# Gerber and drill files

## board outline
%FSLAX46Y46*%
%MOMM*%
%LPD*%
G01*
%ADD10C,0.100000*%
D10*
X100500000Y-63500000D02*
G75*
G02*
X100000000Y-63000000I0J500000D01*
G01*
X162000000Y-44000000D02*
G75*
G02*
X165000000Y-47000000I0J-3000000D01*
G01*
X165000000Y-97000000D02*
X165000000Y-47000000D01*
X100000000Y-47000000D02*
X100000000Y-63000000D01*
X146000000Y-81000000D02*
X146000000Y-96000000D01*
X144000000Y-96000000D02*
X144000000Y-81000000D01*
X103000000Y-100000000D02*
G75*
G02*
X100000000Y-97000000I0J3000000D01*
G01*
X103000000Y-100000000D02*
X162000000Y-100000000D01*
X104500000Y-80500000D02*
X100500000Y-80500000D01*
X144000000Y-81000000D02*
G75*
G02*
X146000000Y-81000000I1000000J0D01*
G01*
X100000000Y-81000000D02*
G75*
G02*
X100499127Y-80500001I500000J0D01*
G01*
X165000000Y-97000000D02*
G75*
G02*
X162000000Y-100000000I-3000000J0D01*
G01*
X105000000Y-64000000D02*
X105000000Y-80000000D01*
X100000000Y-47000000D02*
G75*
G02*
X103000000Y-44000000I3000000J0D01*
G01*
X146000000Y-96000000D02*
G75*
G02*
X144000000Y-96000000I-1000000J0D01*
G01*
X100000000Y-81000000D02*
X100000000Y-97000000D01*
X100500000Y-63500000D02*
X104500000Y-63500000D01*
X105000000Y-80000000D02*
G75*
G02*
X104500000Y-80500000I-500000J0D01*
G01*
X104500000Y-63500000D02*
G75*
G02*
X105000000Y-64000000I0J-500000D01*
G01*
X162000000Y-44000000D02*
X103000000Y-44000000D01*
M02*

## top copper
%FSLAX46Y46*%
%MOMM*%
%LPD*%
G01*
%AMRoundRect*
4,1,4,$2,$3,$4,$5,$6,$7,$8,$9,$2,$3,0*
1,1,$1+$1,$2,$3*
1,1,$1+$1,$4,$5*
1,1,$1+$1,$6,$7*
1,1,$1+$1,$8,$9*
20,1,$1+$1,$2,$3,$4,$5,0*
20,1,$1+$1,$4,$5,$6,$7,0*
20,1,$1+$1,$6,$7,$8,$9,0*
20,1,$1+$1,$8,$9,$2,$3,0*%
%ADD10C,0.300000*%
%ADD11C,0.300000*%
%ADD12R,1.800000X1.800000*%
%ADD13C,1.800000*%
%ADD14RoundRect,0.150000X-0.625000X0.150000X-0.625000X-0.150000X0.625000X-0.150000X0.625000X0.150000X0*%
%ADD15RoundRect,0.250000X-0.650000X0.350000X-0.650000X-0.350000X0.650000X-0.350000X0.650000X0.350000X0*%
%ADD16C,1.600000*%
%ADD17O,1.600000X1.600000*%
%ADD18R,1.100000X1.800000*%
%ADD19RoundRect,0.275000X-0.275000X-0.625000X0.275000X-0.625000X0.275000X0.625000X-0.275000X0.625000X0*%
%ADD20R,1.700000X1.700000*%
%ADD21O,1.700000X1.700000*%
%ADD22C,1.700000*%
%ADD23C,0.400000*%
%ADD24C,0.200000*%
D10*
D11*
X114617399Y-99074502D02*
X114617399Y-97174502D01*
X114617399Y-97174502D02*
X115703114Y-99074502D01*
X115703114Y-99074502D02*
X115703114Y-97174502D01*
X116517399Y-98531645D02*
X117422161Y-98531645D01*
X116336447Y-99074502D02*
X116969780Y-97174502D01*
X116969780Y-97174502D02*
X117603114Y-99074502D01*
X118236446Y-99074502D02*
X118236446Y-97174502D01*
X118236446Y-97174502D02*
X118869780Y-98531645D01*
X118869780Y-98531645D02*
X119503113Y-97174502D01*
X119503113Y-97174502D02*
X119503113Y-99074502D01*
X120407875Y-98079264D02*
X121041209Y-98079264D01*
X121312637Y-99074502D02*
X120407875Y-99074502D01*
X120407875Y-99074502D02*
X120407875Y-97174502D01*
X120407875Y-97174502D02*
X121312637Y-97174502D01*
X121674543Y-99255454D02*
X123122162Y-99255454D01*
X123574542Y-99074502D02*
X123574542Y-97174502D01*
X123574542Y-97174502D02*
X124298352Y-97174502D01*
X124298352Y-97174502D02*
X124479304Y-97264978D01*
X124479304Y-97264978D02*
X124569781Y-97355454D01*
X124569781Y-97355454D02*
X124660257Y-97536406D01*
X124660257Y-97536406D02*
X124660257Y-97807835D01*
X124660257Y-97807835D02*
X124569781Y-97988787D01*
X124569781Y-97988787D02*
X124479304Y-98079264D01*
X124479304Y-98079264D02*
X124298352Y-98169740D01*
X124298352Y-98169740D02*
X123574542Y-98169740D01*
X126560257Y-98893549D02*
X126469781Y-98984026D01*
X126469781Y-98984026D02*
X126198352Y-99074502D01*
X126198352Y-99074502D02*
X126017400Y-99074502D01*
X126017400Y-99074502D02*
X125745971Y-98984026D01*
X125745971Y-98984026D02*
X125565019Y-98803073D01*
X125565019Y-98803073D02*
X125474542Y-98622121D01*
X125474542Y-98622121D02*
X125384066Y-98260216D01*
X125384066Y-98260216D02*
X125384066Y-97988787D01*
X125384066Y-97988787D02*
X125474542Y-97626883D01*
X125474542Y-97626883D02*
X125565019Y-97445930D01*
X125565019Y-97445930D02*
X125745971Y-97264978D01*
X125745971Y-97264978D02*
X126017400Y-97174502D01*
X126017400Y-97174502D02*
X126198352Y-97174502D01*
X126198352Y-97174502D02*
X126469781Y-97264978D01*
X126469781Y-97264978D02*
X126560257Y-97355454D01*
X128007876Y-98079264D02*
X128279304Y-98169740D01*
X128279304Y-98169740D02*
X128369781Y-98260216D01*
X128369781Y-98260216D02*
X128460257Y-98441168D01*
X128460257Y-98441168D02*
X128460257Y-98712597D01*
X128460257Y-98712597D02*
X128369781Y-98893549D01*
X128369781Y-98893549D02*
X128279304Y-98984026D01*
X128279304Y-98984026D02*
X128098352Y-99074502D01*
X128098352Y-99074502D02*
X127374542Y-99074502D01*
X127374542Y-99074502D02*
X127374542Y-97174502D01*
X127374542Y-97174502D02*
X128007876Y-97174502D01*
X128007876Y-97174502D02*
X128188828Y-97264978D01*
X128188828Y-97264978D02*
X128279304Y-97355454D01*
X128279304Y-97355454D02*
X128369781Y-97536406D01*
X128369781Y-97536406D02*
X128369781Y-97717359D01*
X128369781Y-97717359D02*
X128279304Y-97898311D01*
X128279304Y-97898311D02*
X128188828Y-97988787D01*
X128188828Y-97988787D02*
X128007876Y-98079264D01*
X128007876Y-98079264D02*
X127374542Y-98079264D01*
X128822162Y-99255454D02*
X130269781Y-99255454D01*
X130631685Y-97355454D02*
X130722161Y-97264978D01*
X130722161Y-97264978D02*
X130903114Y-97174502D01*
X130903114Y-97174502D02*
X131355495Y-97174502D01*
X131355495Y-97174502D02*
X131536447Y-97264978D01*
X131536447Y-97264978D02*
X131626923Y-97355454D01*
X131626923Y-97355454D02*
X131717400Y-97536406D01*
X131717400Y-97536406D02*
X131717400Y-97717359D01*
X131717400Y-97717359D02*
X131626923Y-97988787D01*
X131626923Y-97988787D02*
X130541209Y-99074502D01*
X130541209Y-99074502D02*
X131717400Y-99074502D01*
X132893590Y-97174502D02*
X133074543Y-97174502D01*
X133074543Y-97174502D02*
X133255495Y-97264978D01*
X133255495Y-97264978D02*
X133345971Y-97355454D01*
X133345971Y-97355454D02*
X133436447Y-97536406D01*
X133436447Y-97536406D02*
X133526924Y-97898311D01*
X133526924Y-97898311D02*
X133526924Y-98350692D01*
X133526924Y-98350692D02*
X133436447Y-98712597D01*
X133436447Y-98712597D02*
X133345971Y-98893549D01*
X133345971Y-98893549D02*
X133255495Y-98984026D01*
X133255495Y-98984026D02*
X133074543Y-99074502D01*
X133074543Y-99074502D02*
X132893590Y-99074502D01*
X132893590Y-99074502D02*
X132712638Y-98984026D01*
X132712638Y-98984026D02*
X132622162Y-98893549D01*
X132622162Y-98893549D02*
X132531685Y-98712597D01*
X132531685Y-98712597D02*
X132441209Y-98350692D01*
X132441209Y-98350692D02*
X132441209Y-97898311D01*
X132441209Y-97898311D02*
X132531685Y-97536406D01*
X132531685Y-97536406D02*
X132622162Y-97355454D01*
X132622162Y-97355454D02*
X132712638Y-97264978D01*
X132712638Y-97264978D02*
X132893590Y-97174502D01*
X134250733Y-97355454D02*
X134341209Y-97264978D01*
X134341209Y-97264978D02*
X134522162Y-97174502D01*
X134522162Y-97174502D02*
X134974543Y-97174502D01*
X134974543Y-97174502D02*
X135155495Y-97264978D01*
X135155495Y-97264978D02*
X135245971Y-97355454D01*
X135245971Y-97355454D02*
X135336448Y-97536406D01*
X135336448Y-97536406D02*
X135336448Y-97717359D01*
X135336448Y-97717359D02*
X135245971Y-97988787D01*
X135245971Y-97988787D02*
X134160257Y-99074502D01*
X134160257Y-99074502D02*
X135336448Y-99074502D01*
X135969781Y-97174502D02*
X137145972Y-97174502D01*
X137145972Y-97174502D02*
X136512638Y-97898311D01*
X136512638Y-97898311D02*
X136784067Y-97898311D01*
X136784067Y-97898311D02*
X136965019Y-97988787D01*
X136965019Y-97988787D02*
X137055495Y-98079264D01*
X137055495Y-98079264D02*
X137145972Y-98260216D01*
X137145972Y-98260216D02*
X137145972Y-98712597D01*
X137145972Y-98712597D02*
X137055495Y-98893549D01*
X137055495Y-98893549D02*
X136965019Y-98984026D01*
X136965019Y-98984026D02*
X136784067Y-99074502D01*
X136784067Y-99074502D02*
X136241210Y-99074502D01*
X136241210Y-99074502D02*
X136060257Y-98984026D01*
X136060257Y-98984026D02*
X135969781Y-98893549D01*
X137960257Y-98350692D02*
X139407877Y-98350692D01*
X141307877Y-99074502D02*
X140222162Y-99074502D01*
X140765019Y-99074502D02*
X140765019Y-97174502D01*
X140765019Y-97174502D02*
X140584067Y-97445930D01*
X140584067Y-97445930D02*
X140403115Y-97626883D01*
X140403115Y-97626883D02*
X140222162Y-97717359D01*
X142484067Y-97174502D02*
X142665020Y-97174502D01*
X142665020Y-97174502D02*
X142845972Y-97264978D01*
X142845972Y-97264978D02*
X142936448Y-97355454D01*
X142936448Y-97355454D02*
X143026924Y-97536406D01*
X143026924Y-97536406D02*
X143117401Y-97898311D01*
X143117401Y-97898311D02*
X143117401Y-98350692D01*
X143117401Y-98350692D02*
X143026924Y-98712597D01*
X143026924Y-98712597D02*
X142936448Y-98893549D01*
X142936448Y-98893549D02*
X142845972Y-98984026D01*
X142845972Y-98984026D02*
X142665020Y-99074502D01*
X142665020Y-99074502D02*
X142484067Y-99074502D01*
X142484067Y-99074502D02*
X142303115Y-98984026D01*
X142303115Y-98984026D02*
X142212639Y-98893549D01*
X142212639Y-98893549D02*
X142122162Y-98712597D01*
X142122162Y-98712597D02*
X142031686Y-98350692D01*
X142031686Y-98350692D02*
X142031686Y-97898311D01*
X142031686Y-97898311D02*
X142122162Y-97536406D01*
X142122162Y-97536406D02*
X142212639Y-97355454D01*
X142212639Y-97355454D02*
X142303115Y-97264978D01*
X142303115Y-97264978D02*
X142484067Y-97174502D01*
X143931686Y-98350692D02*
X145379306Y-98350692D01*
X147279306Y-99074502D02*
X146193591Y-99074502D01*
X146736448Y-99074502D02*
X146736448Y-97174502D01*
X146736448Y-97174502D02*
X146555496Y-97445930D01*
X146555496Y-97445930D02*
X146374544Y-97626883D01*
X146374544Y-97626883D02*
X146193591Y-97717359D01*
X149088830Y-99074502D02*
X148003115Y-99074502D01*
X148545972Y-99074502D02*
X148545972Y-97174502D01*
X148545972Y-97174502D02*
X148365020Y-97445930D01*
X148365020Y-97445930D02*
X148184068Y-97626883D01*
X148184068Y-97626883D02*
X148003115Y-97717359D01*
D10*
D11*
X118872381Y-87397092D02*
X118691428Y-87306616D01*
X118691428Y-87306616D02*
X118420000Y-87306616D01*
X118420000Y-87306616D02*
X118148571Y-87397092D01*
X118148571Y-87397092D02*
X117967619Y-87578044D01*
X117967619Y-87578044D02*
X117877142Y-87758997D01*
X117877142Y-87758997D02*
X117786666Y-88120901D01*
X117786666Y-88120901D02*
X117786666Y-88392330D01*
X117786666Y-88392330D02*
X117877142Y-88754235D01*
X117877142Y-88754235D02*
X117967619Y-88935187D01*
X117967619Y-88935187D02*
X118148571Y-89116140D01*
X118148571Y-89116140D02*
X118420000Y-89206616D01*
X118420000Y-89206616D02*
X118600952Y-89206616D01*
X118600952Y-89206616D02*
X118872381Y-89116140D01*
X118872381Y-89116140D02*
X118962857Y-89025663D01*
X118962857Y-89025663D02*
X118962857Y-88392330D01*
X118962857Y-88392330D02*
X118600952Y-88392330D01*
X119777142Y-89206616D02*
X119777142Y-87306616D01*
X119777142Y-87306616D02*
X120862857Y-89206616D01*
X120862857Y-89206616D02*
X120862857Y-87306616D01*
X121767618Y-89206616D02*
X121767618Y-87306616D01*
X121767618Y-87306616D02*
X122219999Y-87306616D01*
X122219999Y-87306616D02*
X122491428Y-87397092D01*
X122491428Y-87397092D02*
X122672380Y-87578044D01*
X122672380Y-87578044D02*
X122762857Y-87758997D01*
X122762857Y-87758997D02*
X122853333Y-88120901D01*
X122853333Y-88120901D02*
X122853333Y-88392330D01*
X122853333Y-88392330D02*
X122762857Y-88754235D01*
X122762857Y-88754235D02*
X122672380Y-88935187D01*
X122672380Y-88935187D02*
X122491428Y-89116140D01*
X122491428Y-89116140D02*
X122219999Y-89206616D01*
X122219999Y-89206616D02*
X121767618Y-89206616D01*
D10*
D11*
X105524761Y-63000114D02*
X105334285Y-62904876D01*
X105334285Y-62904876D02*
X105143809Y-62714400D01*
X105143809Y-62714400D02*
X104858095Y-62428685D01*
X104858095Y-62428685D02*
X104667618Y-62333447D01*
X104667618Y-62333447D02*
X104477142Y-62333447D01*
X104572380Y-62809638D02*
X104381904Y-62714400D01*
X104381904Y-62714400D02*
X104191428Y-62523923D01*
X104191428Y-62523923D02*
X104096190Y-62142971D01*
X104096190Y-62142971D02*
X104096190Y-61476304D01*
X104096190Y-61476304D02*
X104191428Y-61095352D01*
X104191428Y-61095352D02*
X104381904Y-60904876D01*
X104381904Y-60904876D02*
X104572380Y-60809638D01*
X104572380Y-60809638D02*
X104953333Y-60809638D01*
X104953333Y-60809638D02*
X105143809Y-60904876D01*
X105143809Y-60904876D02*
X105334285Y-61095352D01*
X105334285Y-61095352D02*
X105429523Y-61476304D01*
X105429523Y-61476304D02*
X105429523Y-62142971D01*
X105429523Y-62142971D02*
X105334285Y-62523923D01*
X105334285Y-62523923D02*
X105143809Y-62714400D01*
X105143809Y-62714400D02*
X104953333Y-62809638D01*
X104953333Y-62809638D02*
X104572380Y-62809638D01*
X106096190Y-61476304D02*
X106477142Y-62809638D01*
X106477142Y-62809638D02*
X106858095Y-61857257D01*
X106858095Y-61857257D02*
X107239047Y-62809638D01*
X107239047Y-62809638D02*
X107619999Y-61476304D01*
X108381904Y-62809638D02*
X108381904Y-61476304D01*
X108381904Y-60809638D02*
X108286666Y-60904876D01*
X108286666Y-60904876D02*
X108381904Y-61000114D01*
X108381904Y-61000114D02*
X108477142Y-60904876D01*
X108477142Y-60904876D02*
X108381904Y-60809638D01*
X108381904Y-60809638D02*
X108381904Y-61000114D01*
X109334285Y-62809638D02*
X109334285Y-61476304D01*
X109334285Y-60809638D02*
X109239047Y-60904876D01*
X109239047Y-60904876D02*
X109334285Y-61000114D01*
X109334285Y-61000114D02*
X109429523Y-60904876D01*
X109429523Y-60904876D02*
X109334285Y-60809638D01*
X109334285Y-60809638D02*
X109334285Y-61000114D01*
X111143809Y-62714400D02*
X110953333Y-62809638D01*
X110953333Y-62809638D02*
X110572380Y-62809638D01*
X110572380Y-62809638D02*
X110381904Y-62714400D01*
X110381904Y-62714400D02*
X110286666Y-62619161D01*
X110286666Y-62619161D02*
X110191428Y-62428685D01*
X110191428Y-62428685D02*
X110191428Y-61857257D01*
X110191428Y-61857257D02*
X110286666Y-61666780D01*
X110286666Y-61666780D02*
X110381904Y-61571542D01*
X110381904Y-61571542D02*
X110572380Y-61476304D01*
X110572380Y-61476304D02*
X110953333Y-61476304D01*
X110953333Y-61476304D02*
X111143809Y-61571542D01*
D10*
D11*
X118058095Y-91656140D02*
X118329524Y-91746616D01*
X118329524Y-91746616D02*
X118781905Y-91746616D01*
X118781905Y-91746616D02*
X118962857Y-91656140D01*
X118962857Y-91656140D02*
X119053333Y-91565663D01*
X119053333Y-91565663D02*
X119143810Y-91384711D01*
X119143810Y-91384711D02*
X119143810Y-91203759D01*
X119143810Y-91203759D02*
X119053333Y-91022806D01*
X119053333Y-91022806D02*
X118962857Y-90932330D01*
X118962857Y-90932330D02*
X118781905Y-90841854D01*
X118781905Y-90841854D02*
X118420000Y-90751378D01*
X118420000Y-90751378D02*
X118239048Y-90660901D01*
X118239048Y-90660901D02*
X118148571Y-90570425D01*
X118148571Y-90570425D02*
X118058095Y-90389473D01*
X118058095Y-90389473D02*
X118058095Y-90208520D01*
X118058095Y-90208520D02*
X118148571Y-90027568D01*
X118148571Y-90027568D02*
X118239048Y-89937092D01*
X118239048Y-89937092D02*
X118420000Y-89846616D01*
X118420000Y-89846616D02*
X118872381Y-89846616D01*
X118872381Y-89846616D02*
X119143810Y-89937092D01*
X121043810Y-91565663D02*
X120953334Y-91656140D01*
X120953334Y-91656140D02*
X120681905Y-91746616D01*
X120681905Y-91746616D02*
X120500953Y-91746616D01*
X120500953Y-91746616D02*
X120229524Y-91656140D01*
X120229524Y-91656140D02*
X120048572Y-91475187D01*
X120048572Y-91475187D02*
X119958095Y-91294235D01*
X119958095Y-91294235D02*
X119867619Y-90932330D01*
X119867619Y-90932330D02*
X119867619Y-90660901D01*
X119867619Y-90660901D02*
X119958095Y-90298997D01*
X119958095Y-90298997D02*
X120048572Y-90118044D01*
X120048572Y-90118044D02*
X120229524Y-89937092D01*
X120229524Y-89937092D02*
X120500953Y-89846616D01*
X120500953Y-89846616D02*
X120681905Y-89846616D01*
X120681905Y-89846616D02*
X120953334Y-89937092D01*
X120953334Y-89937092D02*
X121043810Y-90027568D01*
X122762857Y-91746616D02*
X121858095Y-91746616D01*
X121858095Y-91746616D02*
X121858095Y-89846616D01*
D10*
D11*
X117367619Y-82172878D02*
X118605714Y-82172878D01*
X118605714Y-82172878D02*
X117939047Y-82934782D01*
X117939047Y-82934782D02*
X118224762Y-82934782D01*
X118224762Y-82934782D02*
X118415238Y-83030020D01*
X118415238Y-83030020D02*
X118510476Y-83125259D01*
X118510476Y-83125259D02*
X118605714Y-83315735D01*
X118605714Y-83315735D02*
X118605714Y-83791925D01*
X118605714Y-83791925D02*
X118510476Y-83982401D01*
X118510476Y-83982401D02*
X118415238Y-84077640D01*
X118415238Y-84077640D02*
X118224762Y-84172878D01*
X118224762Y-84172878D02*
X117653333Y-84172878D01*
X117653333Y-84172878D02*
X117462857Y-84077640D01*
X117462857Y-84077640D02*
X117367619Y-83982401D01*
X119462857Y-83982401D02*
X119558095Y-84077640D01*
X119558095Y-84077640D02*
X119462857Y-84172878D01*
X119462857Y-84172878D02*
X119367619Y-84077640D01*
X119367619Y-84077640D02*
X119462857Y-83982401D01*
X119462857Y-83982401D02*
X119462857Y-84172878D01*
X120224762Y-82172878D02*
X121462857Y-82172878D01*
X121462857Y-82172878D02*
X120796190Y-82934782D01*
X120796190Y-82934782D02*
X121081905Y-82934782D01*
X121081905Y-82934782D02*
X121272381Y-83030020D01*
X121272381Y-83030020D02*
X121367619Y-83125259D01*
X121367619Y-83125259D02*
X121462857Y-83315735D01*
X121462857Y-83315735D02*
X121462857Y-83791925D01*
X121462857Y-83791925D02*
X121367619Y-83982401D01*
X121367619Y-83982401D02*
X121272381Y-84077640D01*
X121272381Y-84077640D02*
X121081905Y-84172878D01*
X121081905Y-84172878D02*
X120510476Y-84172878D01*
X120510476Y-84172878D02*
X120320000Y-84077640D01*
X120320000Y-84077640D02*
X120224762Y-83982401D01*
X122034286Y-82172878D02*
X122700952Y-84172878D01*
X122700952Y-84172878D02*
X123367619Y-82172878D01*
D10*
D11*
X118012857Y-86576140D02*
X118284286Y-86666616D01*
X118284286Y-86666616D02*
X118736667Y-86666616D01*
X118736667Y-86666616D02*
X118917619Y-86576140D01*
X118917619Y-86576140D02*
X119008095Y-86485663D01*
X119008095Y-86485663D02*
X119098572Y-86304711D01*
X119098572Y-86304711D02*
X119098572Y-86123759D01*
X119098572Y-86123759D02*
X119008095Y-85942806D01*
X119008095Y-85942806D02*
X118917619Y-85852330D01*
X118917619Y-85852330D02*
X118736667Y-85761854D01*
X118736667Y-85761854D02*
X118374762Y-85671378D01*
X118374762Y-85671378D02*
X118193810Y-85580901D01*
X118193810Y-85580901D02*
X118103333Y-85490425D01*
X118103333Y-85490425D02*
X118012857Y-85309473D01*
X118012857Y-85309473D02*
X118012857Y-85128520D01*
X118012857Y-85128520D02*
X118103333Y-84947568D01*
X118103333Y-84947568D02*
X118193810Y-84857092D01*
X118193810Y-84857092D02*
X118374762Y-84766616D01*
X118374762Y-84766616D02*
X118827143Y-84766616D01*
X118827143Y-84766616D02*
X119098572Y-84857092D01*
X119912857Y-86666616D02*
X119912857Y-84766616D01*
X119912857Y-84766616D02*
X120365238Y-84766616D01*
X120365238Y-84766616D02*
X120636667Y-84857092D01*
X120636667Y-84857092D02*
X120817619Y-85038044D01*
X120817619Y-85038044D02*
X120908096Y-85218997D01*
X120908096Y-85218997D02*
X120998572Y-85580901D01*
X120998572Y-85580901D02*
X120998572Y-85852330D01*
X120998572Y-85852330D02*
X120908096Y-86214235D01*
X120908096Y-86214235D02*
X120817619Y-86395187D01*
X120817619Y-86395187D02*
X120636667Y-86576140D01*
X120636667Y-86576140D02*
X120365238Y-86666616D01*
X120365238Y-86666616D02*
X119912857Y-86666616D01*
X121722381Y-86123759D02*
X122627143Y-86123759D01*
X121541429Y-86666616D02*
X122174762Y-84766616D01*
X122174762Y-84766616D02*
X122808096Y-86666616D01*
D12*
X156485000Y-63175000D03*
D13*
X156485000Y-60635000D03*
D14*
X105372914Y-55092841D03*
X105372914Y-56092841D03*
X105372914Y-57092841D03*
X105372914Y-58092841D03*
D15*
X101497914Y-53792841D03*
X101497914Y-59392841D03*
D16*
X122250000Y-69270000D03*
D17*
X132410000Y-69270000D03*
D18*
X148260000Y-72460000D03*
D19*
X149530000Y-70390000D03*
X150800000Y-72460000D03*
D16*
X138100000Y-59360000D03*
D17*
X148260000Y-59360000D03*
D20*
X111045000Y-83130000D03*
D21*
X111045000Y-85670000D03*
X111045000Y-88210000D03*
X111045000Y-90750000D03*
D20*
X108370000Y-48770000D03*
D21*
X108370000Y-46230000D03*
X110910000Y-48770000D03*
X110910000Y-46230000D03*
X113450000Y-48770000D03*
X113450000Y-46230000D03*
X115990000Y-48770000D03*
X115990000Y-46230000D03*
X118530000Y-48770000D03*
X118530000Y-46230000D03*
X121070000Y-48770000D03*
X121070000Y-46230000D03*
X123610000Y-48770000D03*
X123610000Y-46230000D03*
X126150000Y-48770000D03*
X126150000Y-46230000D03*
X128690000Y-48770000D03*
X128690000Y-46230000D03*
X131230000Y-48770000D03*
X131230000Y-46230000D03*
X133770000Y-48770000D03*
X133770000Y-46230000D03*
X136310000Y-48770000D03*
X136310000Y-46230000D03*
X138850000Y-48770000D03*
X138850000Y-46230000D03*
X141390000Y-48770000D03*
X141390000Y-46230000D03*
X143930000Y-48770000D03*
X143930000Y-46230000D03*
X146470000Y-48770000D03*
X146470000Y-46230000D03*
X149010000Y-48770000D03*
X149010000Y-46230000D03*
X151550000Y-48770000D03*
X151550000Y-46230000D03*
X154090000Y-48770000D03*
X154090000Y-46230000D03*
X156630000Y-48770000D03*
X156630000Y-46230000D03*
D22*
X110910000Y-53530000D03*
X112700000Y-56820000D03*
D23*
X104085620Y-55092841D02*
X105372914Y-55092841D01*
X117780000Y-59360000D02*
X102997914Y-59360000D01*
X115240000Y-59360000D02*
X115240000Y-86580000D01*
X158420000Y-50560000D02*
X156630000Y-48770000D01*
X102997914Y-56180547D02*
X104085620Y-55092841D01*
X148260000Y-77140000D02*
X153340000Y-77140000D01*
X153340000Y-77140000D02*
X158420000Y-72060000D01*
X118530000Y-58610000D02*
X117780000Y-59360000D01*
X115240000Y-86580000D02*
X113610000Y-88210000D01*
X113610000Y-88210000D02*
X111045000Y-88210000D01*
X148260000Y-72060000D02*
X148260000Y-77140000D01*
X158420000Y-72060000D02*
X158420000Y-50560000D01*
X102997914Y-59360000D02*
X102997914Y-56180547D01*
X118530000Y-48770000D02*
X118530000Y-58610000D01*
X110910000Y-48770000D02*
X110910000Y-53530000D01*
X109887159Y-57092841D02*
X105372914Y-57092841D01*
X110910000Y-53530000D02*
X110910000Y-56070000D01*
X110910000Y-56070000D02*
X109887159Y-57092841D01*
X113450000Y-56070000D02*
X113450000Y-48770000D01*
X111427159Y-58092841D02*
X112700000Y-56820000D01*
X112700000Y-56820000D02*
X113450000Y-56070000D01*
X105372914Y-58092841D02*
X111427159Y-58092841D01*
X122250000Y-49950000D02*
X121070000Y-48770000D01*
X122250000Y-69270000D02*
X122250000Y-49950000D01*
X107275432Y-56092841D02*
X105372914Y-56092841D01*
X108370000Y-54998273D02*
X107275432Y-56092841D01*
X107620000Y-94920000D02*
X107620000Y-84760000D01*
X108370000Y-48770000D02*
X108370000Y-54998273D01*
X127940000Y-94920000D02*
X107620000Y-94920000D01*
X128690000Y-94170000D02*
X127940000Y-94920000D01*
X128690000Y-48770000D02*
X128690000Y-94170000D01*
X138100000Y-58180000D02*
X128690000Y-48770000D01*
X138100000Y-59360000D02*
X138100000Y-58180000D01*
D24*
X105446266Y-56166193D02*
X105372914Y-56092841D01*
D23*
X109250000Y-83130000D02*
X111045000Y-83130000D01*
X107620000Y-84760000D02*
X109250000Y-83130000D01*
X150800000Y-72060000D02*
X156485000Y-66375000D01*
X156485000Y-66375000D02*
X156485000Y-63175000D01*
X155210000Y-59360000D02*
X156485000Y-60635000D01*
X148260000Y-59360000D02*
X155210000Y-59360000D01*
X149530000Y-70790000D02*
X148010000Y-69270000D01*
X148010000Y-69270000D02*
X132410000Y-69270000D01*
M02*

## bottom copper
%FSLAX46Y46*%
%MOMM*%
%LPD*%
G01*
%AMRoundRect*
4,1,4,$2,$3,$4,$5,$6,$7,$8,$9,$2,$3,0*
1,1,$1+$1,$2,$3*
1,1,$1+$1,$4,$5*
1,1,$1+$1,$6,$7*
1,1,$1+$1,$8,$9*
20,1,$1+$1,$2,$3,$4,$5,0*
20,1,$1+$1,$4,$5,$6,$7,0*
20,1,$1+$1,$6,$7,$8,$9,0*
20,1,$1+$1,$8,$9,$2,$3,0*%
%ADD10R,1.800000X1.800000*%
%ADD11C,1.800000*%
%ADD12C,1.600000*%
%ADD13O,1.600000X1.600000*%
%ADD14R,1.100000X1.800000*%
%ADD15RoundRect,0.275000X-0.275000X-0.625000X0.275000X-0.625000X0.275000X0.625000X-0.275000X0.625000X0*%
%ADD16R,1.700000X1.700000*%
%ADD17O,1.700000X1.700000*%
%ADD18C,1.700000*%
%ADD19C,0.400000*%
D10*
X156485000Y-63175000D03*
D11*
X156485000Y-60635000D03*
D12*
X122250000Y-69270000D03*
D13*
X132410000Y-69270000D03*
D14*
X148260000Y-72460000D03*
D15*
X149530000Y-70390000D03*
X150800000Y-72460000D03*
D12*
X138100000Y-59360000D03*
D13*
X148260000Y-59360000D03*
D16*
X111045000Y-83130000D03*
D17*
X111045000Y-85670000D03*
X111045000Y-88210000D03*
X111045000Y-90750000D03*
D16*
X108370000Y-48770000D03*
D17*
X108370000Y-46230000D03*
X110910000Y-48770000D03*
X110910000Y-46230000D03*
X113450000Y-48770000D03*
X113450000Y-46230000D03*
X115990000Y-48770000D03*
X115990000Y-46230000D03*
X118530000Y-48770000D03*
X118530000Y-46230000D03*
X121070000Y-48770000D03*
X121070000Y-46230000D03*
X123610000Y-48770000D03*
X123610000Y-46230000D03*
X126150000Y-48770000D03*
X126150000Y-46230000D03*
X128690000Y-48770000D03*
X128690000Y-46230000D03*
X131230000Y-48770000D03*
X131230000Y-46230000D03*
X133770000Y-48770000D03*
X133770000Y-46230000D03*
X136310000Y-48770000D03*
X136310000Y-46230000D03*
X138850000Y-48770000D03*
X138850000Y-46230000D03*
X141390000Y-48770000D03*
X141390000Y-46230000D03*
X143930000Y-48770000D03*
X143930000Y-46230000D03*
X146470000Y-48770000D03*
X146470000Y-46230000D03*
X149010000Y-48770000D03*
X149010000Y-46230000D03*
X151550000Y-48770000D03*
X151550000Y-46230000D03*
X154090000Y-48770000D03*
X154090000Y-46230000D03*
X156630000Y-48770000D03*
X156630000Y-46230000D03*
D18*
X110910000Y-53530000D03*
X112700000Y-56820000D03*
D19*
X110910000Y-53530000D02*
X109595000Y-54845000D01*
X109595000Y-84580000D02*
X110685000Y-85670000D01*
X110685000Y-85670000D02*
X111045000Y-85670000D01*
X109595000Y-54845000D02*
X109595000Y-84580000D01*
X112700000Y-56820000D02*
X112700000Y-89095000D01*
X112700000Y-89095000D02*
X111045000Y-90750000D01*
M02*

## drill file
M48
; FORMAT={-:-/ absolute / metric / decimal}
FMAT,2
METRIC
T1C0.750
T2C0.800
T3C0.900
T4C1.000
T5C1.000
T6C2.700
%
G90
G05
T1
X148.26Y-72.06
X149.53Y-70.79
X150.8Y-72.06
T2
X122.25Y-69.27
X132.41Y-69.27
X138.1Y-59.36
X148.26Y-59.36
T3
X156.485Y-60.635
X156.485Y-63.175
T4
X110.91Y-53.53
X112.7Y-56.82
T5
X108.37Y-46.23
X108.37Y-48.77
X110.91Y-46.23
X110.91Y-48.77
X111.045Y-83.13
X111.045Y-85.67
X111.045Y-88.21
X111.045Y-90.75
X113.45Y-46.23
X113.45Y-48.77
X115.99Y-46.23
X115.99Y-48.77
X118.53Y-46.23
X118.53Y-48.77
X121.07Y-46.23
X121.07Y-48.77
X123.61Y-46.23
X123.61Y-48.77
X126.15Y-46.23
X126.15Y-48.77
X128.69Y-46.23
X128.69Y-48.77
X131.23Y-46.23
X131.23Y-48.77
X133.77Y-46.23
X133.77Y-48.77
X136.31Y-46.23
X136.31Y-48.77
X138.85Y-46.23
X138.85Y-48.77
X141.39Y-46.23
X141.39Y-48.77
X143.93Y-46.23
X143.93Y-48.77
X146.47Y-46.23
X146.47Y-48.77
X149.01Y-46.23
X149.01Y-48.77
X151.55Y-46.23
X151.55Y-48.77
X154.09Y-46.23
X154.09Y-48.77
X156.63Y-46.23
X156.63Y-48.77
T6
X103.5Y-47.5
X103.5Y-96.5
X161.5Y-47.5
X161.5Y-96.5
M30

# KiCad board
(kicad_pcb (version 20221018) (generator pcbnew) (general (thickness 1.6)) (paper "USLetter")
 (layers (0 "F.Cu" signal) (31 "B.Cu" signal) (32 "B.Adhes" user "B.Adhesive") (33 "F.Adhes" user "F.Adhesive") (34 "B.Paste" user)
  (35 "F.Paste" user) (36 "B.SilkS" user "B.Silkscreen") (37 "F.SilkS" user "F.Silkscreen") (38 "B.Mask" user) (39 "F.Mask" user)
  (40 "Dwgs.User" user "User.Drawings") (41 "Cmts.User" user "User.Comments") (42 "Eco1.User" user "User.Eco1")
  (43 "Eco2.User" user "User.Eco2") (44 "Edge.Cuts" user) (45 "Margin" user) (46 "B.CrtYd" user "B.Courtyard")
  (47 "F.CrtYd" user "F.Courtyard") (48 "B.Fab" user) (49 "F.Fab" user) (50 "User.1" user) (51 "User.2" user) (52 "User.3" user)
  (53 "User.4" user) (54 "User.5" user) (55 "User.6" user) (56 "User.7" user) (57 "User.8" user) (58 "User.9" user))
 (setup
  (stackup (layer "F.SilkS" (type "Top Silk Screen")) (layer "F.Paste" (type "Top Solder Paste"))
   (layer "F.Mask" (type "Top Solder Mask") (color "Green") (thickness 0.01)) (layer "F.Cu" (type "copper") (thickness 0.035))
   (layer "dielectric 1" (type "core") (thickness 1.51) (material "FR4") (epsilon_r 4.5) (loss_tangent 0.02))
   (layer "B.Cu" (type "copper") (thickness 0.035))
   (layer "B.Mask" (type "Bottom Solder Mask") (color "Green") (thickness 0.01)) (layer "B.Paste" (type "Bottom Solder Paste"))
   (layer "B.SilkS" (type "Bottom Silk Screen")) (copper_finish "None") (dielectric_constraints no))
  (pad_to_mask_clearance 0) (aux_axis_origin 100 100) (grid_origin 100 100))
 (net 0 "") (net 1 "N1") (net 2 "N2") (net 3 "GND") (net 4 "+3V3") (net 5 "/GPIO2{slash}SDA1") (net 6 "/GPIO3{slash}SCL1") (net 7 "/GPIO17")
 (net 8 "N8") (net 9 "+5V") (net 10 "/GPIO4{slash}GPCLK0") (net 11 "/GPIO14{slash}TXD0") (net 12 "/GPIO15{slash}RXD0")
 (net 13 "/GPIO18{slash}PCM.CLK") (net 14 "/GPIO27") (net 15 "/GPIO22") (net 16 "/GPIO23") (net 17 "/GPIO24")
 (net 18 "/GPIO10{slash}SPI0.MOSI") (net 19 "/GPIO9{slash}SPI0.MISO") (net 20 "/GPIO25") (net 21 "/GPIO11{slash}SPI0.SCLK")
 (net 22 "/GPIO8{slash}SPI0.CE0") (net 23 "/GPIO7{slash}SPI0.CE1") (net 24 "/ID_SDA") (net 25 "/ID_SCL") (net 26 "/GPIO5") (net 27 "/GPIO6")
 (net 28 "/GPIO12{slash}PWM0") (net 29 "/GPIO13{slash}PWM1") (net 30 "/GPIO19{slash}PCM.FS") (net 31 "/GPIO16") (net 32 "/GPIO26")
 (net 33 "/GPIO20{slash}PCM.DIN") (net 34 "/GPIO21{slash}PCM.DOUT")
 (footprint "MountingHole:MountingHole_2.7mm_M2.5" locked (layer "F.Cu") (at 161.5 47.5)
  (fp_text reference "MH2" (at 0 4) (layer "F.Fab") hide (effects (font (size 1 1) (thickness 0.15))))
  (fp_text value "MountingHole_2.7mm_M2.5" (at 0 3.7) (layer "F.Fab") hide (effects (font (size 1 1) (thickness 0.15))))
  (pad "" np_thru_hole circle locked (at 0 0) (size 2.7 2.7) (drill 2.7) (layers "*.Cu" "*.Mask")))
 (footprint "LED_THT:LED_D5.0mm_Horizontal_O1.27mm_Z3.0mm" (layer "F.Cu") (at 156.485 63.175 90)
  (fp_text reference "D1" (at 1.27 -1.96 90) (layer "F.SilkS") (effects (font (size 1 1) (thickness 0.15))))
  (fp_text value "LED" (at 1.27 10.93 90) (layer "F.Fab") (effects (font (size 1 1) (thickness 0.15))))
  (pad "1" thru_hole rect (at 0 0 90) (size 1.8 1.8) (drill 0.9) (layers "*.Cu" "*.Mask") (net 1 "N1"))
  (pad "2" thru_hole circle (at 2.54 0 90) (size 1.8 1.8) (drill 0.9) (layers "*.Cu" "*.Mask") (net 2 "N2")))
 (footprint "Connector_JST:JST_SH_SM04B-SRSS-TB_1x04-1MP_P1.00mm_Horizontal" (layer "F.Cu") (at 103.372914 56.592841 -90)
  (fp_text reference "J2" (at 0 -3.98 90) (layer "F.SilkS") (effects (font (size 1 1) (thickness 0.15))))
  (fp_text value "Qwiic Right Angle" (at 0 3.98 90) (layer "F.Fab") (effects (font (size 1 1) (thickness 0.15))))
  (pad "1" smd roundrect (at -1.5 -2 270) (size 0.6 1.55) (layers "F.Cu" "F.Paste" "F.Mask") (roundrect_rratio 0.25) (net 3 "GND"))
  (pad "2" smd roundrect (at -0.5 -2 270) (size 0.6 1.55) (layers "F.Cu" "F.Paste" "F.Mask") (roundrect_rratio 0.25) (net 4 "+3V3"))
  (pad "3" smd roundrect (at 0.5 -2 270) (size 0.6 1.55) (layers "F.Cu" "F.Paste" "F.Mask") (roundrect_rratio 0.25)
   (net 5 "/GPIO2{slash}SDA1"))
  (pad "4" smd roundrect (at 1.5 -2 270) (size 0.6 1.55) (layers "F.Cu" "F.Paste" "F.Mask") (roundrect_rratio 0.25)
   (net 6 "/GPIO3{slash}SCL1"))
  (pad "MP" smd roundrect (at -2.8 1.875 270) (size 1.2 1.8) (layers "F.Cu" "F.Paste" "F.Mask") (roundrect_rratio 0.2083333333))
  (pad "MP" smd roundrect (at 2.8 1.875 270) (size 1.2 1.8) (layers "F.Cu" "F.Paste" "F.Mask") (roundrect_rratio 0.2083333333)))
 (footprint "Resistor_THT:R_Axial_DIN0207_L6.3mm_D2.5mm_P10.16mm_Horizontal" (layer "F.Cu") (at 122.25 69.27)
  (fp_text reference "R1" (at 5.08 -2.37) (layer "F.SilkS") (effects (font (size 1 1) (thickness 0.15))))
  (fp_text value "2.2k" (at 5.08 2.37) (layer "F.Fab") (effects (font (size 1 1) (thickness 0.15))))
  (pad "1" thru_hole circle (at 0 0) (size 1.6 1.6) (drill 0.8) (layers "*.Cu" "*.Mask") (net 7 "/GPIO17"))
  (pad "2" thru_hole oval (at 10.16 0) (size 1.6 1.6) (drill 0.8) (layers "*.Cu" "*.Mask") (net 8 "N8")))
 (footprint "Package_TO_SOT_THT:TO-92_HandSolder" (layer "F.Cu") (at 148.26 72.06)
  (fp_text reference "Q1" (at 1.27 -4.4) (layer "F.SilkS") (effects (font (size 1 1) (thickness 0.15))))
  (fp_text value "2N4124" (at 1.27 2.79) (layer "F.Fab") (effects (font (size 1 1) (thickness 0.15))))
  (pad "1" thru_hole rect (at 0 0) (size 1.1 1.8) (drill 0.75 (offset 0 0.4)) (layers "*.Cu" "*.Mask") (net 3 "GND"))
  (pad "2" thru_hole roundrect (at 1.27 -1.27) (size 1.1 1.8) (drill 0.75 (offset 0 -0.4)) (layers "*.Cu" "*.Mask") (roundrect_rratio 0.25)
   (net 8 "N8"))
  (pad "3" thru_hole roundrect (at 2.54 0) (size 1.1 1.8) (drill 0.75 (offset 0 0.4)) (layers "*.Cu" "*.Mask") (roundrect_rratio 0.25)
   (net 1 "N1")))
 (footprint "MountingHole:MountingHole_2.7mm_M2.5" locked (layer "F.Cu") (at 103.5 96.5)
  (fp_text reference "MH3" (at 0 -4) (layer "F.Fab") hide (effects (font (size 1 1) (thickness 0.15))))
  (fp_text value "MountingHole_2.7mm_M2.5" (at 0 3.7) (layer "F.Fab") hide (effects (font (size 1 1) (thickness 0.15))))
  (pad "" np_thru_hole circle locked (at 0 0) (size 2.7 2.7) (drill 2.7) (layers "*.Cu" "*.Mask")))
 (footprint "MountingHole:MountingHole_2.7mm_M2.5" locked (layer "F.Cu") (at 103.5 47.5)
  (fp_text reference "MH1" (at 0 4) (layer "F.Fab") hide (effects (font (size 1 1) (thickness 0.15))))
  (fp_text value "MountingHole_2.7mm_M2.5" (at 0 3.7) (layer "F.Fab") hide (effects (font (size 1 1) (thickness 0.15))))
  (pad "" np_thru_hole circle locked (at 0 0) (size 2.7 2.7) (drill 2.7) (layers "*.Cu" "*.Mask")))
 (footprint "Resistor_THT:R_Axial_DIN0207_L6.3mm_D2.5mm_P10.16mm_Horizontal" (layer "F.Cu") (at 138.1 59.36)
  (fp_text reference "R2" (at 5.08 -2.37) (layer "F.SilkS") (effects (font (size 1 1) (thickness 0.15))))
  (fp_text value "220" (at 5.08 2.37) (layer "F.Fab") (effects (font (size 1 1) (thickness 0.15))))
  (pad "1" thru_hole circle (at 0 0) (size 1.6 1.6) (drill 0.8) (layers "*.Cu" "*.Mask") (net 4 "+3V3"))
  (pad "2" thru_hole oval (at 10.16 0) (size 1.6 1.6) (drill 0.8) (layers "*.Cu" "*.Mask") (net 2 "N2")))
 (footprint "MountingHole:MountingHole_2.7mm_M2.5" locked (layer "F.Cu") (at 161.5 96.5)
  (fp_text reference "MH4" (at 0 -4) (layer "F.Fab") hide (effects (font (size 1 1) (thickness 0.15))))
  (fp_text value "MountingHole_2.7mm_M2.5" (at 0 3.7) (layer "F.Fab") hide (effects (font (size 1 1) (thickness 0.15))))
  (pad "" np_thru_hole circle locked (at 0 0) (size 2.7 2.7) (drill 2.7) (layers "*.Cu" "*.Mask")))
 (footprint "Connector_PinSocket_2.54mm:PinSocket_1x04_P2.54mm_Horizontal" (layer "F.Cu") (at 111.045 83.13)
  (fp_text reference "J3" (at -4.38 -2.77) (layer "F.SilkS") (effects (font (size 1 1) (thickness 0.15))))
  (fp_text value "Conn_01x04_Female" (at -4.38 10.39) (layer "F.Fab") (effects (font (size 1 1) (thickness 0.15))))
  (pad "1" thru_hole rect (at 0 0) (size 1.7 1.7) (drill 1) (layers "*.Cu" "*.Mask") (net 4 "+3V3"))
  (pad "2" thru_hole oval (at 0 2.54) (size 1.7 1.7) (drill 1) (layers "*.Cu" "*.Mask") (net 5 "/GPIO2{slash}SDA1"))
  (pad "3" thru_hole oval (at 0 5.08) (size 1.7 1.7) (drill 1) (layers "*.Cu" "*.Mask") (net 3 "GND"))
  (pad "4" thru_hole oval (at 0 7.62) (size 1.7 1.7) (drill 1) (layers "*.Cu" "*.Mask") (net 6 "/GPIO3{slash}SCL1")))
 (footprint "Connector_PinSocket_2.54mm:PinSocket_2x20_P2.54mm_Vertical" (layer "B.Cu") (at 108.37 48.77 -90)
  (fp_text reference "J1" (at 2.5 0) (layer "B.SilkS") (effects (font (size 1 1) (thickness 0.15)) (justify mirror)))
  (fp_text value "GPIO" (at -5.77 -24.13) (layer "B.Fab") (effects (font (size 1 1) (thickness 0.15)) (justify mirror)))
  (pad "1" thru_hole rect (at 0 0 270) (size 1.7 1.7) (drill 1) (layers "*.Cu" "*.Mask") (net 4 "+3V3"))
  (pad "2" thru_hole oval (at -2.54 0 270) (size 1.7 1.7) (drill 1) (layers "*.Cu" "*.Mask") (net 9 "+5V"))
  (pad "3" thru_hole oval (at 0 -2.54 270) (size 1.7 1.7) (drill 1) (layers "*.Cu" "*.Mask") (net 5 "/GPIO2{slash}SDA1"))
  (pad "4" thru_hole oval (at -2.54 -2.54 270) (size 1.7 1.7) (drill 1) (layers "*.Cu" "*.Mask") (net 9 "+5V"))
  (pad "5" thru_hole oval (at 0 -5.08 270) (size 1.7 1.7) (drill 1) (layers "*.Cu" "*.Mask") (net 6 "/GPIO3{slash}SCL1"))
  (pad "6" thru_hole oval (at -2.54 -5.08 270) (size 1.7 1.7) (drill 1) (layers "*.Cu" "*.Mask") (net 3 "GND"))
  (pad "7" thru_hole oval (at 0 -7.62 270) (size 1.7 1.7) (drill 1) (layers "*.Cu" "*.Mask") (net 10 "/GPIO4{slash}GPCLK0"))
  (pad "8" thru_hole oval (at -2.54 -7.62 270) (size 1.7 1.7) (drill 1) (layers "*.Cu" "*.Mask") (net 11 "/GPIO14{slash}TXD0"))
  (pad "9" thru_hole oval (at 0 -10.16 270) (size 1.7 1.7) (drill 1) (layers "*.Cu" "*.Mask") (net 3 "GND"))
  (pad "10" thru_hole oval (at -2.54 -10.16 270) (size 1.7 1.7) (drill 1) (layers "*.Cu" "*.Mask") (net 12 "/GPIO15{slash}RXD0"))
  (pad "11" thru_hole oval (at 0 -12.7 270) (size 1.7 1.7) (drill 1) (layers "*.Cu" "*.Mask") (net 7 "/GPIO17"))
  (pad "12" thru_hole oval (at -2.54 -12.7 270) (size 1.7 1.7) (drill 1) (layers "*.Cu" "*.Mask") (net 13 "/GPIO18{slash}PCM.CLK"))
  (pad "13" thru_hole oval (at 0 -15.24 270) (size 1.7 1.7) (drill 1) (layers "*.Cu" "*.Mask") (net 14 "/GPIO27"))
  (pad "14" thru_hole oval (at -2.54 -15.24 270) (size 1.7 1.7) (drill 1) (layers "*.Cu" "*.Mask") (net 3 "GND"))
  (pad "15" thru_hole oval (at 0 -17.78 270) (size 1.7 1.7) (drill 1) (layers "*.Cu" "*.Mask") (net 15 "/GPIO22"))
  (pad "16" thru_hole oval (at -2.54 -17.78 270) (size 1.7 1.7) (drill 1) (layers "*.Cu" "*.Mask") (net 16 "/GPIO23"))
  (pad "17" thru_hole oval (at 0 -20.32 270) (size 1.7 1.7) (drill 1) (layers "*.Cu" "*.Mask") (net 4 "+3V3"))
  (pad "18" thru_hole oval (at -2.54 -20.32 270) (size 1.7 1.7) (drill 1) (layers "*.Cu" "*.Mask") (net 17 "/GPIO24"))
  (pad "19" thru_hole oval (at 0 -22.86 270) (size 1.7 1.7) (drill 1) (layers "*.Cu" "*.Mask") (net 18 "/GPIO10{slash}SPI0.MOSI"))
  (pad "20" thru_hole oval (at -2.54 -22.86 270) (size 1.7 1.7) (drill 1) (layers "*.Cu" "*.Mask") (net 3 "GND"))
  (pad "21" thru_hole oval (at 0 -25.4 270) (size 1.7 1.7) (drill 1) (layers "*.Cu" "*.Mask") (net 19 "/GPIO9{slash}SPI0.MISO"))
  (pad "22" thru_hole oval (at -2.54 -25.4 270) (size 1.7 1.7) (drill 1) (layers "*.Cu" "*.Mask") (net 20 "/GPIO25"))
  (pad "23" thru_hole oval (at 0 -27.94 270) (size 1.7 1.7) (drill 1) (layers "*.Cu" "*.Mask") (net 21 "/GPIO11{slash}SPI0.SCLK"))
  (pad "24" thru_hole oval (at -2.54 -27.94 270) (size 1.7 1.7) (drill 1) (layers "*.Cu" "*.Mask") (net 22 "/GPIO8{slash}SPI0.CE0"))
  (pad "25" thru_hole oval (at 0 -30.48 270) (size 1.7 1.7) (drill 1) (layers "*.Cu" "*.Mask") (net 3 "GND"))
  (pad "26" thru_hole oval (at -2.54 -30.48 270) (size 1.7 1.7) (drill 1) (layers "*.Cu" "*.Mask") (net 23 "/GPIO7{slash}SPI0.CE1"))
  (pad "27" thru_hole oval (at 0 -33.02 270) (size 1.7 1.7) (drill 1) (layers "*.Cu" "*.Mask") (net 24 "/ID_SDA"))
  (pad "28" thru_hole oval (at -2.54 -33.02 270) (size 1.7 1.7) (drill 1) (layers "*.Cu" "*.Mask") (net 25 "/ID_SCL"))
  (pad "29" thru_hole oval (at 0 -35.56 270) (size 1.7 1.7) (drill 1) (layers "*.Cu" "*.Mask") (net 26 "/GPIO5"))
  (pad "30" thru_hole oval (at -2.54 -35.56 270) (size 1.7 1.7) (drill 1) (layers "*.Cu" "*.Mask") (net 3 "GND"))
  (pad "31" thru_hole oval (at 0 -38.1 270) (size 1.7 1.7) (drill 1) (layers "*.Cu" "*.Mask") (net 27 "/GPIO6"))
  (pad "32" thru_hole oval (at -2.54 -38.1 270) (size 1.7 1.7) (drill 1) (layers "*.Cu" "*.Mask") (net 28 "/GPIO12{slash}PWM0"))
  (pad "33" thru_hole oval (at 0 -40.64 270) (size 1.7 1.7) (drill 1) (layers "*.Cu" "*.Mask") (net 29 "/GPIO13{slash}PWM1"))
  (pad "34" thru_hole oval (at -2.54 -40.64 270) (size 1.7 1.7) (drill 1) (layers "*.Cu" "*.Mask") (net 3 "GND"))
  (pad "35" thru_hole oval (at 0 -43.18 270) (size 1.7 1.7) (drill 1) (layers "*.Cu" "*.Mask") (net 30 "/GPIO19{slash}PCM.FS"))
  (pad "36" thru_hole oval (at -2.54 -43.18 270) (size 1.7 1.7) (drill 1) (layers "*.Cu" "*.Mask") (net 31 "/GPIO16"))
  (pad "37" thru_hole oval (at 0 -45.72 270) (size 1.7 1.7) (drill 1) (layers "*.Cu" "*.Mask") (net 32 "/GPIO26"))
  (pad "38" thru_hole oval (at -2.54 -45.72 270) (size 1.7 1.7) (drill 1) (layers "*.Cu" "*.Mask") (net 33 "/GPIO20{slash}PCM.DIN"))
  (pad "39" thru_hole oval (at 0 -48.26 270) (size 1.7 1.7) (drill 1) (layers "*.Cu" "*.Mask") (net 3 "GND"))
  (pad "40" thru_hole oval (at -2.54 -48.26 270) (size 1.7 1.7) (drill 1) (layers "*.Cu" "*.Mask") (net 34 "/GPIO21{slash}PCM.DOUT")))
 (gr_arc (start 100.5 63.5) (mid 100.146447 63.353553) (end 100 63) (stroke (width 0.1) (type solid)) (layer "Edge.Cuts"))
 (gr_arc (start 162 44) (mid 164.12132 44.87868) (end 165 47) (stroke (width 0.1) (type solid)) (layer "Edge.Cuts"))
 (gr_line (start 165 97) (end 165 47) (stroke (width 0.1) (type solid)) (layer "Edge.Cuts"))
 (gr_line (start 100 47) (end 100 63) (stroke (width 0.1) (type solid)) (layer "Edge.Cuts"))
 (gr_line (start 146 81) (end 146 96) (stroke (width 0.1) (type solid)) (layer "Edge.Cuts"))
 (gr_line (start 144 96) (end 144 81) (stroke (width 0.1) (type solid)) (layer "Edge.Cuts"))
 (gr_arc (start 103 100) (mid 100.87868 99.12132) (end 100 97) (stroke (width 0.1) (type solid)) (layer "Edge.Cuts"))
 (gr_line (start 103 100) (end 162 100) (stroke (width 0.1) (type solid)) (layer "Edge.Cuts"))
 (gr_line (start 104.5 80.5) (end 100.5 80.5) (stroke (width 0.1) (type solid)) (layer "Edge.Cuts"))
 (gr_arc (start 144 81) (mid 145 80) (end 146 81) (stroke (width 0.1) (type solid)) (layer "Edge.Cuts"))
 (gr_arc (start 100 81) (mid 100.146138 80.646755) (end 100.499127 80.500001) (stroke (width 0.1) (type solid)) (layer "Edge.Cuts"))
 (gr_arc (start 165 97) (mid 164.12132 99.12132) (end 162 100) (stroke (width 0.1) (type solid)) (layer "Edge.Cuts"))
 (gr_line (start 105 64) (end 105 80) (stroke (width 0.1) (type solid)) (layer "Edge.Cuts"))
 (gr_arc (start 100 47) (mid 100.87868 44.87868) (end 103 44) (stroke (width 0.1) (type solid)) (layer "Edge.Cuts"))
 (gr_arc (start 146 96) (mid 145 97) (end 144 96) (stroke (width 0.1) (type solid)) (layer "Edge.Cuts"))
 (gr_line (start 100 81) (end 100 97) (stroke (width 0.1) (type solid)) (layer "Edge.Cuts"))
 (gr_line (start 100.5 63.5) (end 104.5 63.5) (stroke (width 0.1) (type solid)) (layer "Edge.Cuts"))
 (gr_arc (start 105 80) (mid 104.853553 80.353553) (end 104.5 80.5) (stroke (width 0.1) (type solid)) (layer "Edge.Cuts"))
 (gr_arc (start 104.5 63.5) (mid 104.853553 63.646447) (end 105 64) (stroke (width 0.1) (type solid)) (layer "Edge.Cuts"))
 (gr_line (start 162 44) (end 103 44) (stroke (width 0.1) (type solid)) (layer "Edge.Cuts"))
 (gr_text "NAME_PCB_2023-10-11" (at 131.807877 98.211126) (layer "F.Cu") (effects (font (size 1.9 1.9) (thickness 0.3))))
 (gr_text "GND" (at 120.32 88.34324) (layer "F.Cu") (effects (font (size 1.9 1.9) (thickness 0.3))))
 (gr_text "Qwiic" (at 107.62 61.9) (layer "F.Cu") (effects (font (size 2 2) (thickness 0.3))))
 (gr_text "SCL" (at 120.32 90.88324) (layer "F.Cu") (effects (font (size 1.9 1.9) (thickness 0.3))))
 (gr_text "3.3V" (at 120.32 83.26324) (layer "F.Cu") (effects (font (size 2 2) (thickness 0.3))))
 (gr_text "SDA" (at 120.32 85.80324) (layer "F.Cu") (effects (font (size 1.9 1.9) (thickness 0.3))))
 (segment (start 104.08562 55.092841) (end 105.372914 55.092841) (width 0.4) (layer "F.Cu") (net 3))
 (segment (start 117.78 59.36) (end 102.997914 59.36) (width 0.4) (layer "F.Cu") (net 3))
 (segment (start 115.24 59.36) (end 115.24 86.58) (width 0.4) (layer "F.Cu") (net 3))
 (segment (start 158.42 50.56) (end 156.63 48.77) (width 0.4) (layer "F.Cu") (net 3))
 (segment (start 102.997914 56.180547) (end 104.08562 55.092841) (width 0.4) (layer "F.Cu") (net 3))
 (segment (start 148.26 77.14) (end 153.34 77.14) (width 0.4) (layer "F.Cu") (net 3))
 (segment (start 153.34 77.14) (end 158.42 72.06) (width 0.4) (layer "F.Cu") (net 3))
 (segment (start 118.53 58.61) (end 117.78 59.36) (width 0.4) (layer "F.Cu") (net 3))
 (segment (start 115.24 86.58) (end 113.61 88.21) (width 0.4) (layer "F.Cu") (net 3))
 (segment (start 113.61 88.21) (end 111.045 88.21) (width 0.4) (layer "F.Cu") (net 3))
 (segment (start 148.26 72.06) (end 148.26 77.14) (width 0.4) (layer "F.Cu") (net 3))
 (segment (start 158.42 72.06) (end 158.42 50.56) (width 0.4) (layer "F.Cu") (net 3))
 (segment (start 102.997914 59.36) (end 102.997914 56.180547) (width 0.4) (layer "F.Cu") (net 3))
 (segment (start 118.53 48.77) (end 118.53 58.61) (width 0.4) (layer "F.Cu") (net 3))
 (segment (start 110.91 48.77) (end 110.91 53.53) (width 0.4) (layer "F.Cu") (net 5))
 (segment (start 109.887159 57.092841) (end 105.372914 57.092841) (width 0.4) (layer "F.Cu") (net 5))
 (segment (start 110.91 53.53) (end 110.91 56.07) (width 0.4) (layer "F.Cu") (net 5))
 (segment (start 110.91 56.07) (end 109.887159 57.092841) (width 0.4) (layer "F.Cu") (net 5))
 (via (at 110.91 53.53) (size 1.7) (drill 1) (layers "F.Cu" "B.Cu") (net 5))
 (segment (start 110.91 53.53) (end 109.595 54.845) (width 0.4) (layer "B.Cu") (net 5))
 (segment (start 109.595 84.58) (end 110.685 85.67) (width 0.4) (layer "B.Cu") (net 5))
 (segment (start 110.685 85.67) (end 111.045 85.67) (width 0.4) (layer "B.Cu") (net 5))
 (segment (start 109.595 54.845) (end 109.595 84.58) (width 0.4) (layer "B.Cu") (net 5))
 (segment (start 113.45 56.07) (end 113.45 48.77) (width 0.4) (layer "F.Cu") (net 6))
 (segment (start 111.427159 58.092841) (end 112.7 56.82) (width 0.4) (layer "F.Cu") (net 6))
 (segment (start 112.7 56.82) (end 113.45 56.07) (width 0.4) (layer "F.Cu") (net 6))
 (segment (start 105.372914 58.092841) (end 111.427159 58.092841) (width 0.4) (layer "F.Cu") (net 6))
 (via (at 112.7 56.82) (size 1.7) (drill 1) (layers "F.Cu" "B.Cu") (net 6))
 (segment (start 112.7 56.82) (end 112.7 89.095) (width 0.4) (layer "B.Cu") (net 6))
 (segment (start 112.7 89.095) (end 111.045 90.75) (width 0.4) (layer "B.Cu") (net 6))
 (segment (start 122.25 49.95) (end 121.07 48.77) (width 0.4) (layer "F.Cu") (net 7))
 (segment (start 122.25 69.27) (end 122.25 49.95) (width 0.4) (layer "F.Cu") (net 7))
 (segment (start 107.275432 56.092841) (end 105.372914 56.092841) (width 0.4) (layer "F.Cu") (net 4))
 (segment (start 108.37 54.998273) (end 107.275432 56.092841) (width 0.4) (layer "F.Cu") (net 4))
 (segment (start 107.62 94.92) (end 107.62 84.76) (width 0.4) (layer "F.Cu") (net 4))
 (segment (start 108.37 48.77) (end 108.37 54.998273) (width 0.4) (layer "F.Cu") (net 4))
 (segment (start 127.94 94.92) (end 107.62 94.92) (width 0.4) (layer "F.Cu") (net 4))
 (segment (start 128.69 94.17) (end 127.94 94.92) (width 0.4) (layer "F.Cu") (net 4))
 (segment (start 128.69 48.77) (end 128.69 94.17) (width 0.4) (layer "F.Cu") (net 4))
 (segment (start 138.1 58.18) (end 128.69 48.77) (width 0.4) (layer "F.Cu") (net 4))
 (segment (start 138.1 59.36) (end 138.1 58.18) (width 0.4) (layer "F.Cu") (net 4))
 (segment (start 105.446266 56.166193) (end 105.372914 56.092841) (width 0.2) (layer "F.Cu") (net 4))
 (segment (start 109.25 83.13) (end 111.045 83.13) (width 0.4) (layer "F.Cu") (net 4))
 (segment (start 107.62 84.76) (end 109.25 83.13) (width 0.4) (layer "F.Cu") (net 4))
 (segment (start 150.8 72.06) (end 156.485 66.375) (width 0.4) (layer "F.Cu") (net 1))
 (segment (start 156.485 66.375) (end 156.485 63.175) (width 0.4) (layer "F.Cu") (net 1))
 (segment (start 155.21 59.36) (end 156.485 60.635) (width 0.4) (layer "F.Cu") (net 2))
 (segment (start 148.26 59.36) (end 155.21 59.36) (width 0.4) (layer "F.Cu") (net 2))
 (segment (start 149.53 70.79) (end 148.01 69.27) (width 0.4) (layer "F.Cu") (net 8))
 (segment (start 148.01 69.27) (end 132.41 69.27) (width 0.4) (layer "F.Cu") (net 8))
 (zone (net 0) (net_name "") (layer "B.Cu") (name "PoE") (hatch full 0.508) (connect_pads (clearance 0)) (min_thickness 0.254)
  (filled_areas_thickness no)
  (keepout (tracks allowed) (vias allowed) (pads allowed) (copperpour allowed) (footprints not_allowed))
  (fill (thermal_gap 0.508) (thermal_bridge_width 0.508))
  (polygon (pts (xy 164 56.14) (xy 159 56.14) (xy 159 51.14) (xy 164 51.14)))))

